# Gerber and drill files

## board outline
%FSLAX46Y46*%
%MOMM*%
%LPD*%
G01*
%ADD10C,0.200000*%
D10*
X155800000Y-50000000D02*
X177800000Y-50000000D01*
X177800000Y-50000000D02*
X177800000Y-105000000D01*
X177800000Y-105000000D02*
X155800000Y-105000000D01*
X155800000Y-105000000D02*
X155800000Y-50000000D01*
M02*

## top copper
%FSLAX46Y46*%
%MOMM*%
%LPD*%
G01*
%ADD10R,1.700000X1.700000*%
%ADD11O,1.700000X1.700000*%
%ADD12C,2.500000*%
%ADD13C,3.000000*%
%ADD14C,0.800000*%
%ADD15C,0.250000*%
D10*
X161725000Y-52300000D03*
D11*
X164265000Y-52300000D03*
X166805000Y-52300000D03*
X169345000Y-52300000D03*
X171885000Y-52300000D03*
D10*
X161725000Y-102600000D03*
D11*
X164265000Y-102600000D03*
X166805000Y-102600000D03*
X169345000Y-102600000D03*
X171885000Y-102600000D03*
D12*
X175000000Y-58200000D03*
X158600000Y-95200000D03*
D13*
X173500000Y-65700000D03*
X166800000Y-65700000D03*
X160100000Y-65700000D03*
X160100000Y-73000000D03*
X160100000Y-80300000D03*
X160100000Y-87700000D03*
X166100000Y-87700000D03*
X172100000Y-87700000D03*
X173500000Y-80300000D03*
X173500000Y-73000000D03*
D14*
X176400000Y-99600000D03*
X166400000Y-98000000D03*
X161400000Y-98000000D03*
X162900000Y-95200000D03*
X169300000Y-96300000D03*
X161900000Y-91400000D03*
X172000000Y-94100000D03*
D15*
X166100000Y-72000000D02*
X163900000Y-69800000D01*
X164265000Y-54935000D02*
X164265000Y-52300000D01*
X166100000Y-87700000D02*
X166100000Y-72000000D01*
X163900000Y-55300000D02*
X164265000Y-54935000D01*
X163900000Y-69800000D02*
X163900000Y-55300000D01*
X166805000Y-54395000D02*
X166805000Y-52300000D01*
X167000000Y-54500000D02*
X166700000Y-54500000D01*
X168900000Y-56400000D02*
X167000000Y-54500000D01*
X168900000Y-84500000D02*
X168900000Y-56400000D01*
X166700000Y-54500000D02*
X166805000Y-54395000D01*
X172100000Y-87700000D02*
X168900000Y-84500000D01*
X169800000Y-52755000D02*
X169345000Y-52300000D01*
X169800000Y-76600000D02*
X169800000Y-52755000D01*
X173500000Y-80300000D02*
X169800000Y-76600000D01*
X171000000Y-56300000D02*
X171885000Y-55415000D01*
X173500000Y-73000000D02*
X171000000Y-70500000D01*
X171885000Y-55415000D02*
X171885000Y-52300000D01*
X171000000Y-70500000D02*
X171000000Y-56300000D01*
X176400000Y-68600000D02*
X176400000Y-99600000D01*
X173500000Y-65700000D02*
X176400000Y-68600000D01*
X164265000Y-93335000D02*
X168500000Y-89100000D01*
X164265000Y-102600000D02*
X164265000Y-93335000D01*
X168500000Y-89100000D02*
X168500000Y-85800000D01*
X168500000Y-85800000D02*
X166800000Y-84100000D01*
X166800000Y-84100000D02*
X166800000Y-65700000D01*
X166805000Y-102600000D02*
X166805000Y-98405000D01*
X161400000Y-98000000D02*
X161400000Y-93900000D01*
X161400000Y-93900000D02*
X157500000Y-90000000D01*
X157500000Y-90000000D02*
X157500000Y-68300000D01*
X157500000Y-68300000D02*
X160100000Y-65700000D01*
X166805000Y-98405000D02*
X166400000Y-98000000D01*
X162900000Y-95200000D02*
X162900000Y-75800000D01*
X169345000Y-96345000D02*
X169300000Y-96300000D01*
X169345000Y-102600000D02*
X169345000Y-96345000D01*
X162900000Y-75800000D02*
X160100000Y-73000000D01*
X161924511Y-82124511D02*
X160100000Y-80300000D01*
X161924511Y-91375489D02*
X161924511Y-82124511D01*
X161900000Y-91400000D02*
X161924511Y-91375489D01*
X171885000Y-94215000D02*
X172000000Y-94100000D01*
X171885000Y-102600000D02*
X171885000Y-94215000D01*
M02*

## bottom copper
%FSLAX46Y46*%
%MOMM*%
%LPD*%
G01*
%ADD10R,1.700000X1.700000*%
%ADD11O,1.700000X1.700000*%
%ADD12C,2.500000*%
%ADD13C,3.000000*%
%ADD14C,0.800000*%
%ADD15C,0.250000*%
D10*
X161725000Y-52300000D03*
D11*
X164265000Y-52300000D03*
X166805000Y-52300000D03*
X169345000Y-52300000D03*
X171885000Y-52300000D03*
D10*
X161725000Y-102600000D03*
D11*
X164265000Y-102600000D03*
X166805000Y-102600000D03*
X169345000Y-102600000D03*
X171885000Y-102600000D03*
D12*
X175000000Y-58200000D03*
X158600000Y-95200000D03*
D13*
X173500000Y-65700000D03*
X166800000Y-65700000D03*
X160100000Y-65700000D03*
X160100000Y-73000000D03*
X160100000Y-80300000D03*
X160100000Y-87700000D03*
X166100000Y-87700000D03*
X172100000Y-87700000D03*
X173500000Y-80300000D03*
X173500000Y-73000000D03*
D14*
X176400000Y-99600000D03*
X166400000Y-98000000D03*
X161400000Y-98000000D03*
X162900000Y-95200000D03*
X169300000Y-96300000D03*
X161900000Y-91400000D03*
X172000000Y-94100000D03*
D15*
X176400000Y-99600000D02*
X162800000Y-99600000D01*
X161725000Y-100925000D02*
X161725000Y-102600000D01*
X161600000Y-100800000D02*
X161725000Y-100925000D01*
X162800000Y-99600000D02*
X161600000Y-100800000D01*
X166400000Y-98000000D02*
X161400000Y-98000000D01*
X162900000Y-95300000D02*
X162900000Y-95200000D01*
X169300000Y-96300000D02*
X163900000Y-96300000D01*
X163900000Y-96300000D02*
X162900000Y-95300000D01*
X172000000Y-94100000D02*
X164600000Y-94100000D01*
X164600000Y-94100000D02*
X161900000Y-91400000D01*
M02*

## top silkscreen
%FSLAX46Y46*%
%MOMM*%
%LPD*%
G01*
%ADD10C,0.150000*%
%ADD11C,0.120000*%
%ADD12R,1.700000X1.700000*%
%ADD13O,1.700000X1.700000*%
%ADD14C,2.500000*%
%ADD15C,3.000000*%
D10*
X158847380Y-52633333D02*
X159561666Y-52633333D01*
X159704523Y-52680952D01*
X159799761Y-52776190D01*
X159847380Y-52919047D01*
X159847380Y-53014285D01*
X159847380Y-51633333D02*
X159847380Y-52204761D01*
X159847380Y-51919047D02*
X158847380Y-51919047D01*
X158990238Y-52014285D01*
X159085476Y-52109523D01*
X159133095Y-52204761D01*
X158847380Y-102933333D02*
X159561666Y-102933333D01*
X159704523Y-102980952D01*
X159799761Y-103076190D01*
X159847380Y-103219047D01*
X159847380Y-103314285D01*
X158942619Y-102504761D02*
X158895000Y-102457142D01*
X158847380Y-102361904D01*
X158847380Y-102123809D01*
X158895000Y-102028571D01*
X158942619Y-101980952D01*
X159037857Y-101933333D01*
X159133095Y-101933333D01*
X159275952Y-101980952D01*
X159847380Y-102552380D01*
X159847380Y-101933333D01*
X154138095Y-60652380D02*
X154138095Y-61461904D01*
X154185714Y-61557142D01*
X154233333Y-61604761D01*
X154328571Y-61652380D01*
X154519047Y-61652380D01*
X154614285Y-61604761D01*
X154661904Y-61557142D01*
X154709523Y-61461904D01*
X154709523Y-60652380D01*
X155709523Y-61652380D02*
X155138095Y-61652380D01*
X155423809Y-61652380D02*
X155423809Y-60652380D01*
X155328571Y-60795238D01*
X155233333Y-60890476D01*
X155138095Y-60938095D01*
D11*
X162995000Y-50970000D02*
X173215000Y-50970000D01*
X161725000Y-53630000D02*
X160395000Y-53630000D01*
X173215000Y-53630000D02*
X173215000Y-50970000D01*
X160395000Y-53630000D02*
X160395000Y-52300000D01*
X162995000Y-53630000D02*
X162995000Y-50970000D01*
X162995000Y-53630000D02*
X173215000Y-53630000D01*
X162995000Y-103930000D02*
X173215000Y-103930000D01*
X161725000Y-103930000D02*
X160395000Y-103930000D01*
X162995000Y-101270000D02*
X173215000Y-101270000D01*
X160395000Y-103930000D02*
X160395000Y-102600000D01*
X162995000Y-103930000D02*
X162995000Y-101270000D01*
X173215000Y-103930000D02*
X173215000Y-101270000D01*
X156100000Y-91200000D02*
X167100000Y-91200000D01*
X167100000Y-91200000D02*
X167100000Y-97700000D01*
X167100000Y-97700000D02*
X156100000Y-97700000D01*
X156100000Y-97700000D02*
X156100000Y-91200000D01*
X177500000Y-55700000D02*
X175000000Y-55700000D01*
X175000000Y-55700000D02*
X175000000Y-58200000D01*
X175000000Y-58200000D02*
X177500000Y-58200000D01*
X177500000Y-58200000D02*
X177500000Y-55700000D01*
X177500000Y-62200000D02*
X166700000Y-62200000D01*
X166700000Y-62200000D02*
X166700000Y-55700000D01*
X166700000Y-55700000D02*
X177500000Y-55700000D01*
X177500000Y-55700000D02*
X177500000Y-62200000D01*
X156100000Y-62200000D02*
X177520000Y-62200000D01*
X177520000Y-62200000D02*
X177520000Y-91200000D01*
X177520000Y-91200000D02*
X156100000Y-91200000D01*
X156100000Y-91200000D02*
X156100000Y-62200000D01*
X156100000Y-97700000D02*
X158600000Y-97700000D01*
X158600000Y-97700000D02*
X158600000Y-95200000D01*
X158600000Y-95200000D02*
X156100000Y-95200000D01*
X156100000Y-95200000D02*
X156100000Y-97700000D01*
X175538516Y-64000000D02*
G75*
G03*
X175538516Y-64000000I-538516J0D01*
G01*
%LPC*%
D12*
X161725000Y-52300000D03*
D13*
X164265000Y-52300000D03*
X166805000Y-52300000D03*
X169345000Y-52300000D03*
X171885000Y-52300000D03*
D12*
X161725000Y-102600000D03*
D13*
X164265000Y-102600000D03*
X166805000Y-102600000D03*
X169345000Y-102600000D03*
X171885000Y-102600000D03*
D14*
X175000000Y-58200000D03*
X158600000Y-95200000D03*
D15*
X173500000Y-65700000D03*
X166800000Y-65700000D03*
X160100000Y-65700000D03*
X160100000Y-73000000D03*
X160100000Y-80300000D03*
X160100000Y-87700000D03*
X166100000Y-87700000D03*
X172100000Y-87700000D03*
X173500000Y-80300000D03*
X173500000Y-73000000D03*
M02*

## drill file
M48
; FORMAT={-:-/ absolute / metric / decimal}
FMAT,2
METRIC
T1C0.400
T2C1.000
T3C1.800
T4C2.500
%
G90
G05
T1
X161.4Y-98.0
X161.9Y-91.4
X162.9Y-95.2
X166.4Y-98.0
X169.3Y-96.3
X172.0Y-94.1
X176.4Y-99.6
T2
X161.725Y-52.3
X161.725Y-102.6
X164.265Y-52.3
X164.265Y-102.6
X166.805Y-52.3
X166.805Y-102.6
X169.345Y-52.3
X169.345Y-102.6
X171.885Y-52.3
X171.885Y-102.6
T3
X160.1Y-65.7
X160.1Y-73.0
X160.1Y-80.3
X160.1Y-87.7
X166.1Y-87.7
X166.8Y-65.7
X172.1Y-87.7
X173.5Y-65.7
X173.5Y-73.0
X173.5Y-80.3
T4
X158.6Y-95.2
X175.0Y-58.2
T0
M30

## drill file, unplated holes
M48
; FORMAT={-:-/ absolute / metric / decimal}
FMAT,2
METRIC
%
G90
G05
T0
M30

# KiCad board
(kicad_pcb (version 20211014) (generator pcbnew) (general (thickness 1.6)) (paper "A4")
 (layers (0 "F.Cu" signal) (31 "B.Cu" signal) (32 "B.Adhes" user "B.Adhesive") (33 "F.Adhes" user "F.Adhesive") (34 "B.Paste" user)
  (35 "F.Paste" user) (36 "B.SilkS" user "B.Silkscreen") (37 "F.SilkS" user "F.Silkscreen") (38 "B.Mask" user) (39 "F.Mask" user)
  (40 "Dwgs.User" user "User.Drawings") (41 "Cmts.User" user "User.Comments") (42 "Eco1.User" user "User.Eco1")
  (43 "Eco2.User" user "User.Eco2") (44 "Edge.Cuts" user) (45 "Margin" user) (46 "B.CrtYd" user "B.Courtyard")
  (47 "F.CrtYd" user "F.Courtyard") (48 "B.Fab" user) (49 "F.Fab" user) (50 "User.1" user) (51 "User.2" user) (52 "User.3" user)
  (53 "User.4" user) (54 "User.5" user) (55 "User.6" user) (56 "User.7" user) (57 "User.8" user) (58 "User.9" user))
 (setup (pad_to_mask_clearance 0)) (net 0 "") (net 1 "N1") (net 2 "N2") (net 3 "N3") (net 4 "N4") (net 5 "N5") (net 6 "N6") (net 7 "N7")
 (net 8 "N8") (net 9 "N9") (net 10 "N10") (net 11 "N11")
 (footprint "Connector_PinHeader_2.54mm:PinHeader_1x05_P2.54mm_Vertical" (layer "F.Cu") (at 161.725 52.3 90)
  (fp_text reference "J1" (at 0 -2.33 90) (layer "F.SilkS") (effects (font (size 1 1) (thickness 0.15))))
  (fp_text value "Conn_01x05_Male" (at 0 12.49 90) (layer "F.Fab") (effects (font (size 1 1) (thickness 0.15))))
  (fp_line (start 1.33 1.27) (end 1.33 11.49) (layer "F.SilkS") (width 0.12))
  (fp_line (start -1.33 0) (end -1.33 -1.33) (layer "F.SilkS") (width 0.12))
  (fp_line (start -1.33 11.49) (end 1.33 11.49) (layer "F.SilkS") (width 0.12))
  (fp_line (start -1.33 -1.33) (end 0 -1.33) (layer "F.SilkS") (width 0.12))
  (fp_line (start -1.33 1.27) (end 1.33 1.27) (layer "F.SilkS") (width 0.12))
  (fp_line (start -1.33 1.27) (end -1.33 11.49) (layer "F.SilkS") (width 0.12))
  (pad "1" thru_hole rect (at 0 0 90) (size 1.7 1.7) (drill 1) (layers *.Cu *.Mask) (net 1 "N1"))
  (pad "2" thru_hole oval (at 0 2.54 90) (size 1.7 1.7) (drill 1) (layers *.Cu *.Mask) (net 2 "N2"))
  (pad "3" thru_hole oval (at 0 5.08 90) (size 1.7 1.7) (drill 1) (layers *.Cu *.Mask) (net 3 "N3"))
  (pad "4" thru_hole oval (at 0 7.62 90) (size 1.7 1.7) (drill 1) (layers *.Cu *.Mask) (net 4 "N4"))
  (pad "5" thru_hole oval (at 0 10.16 90) (size 1.7 1.7) (drill 1) (layers *.Cu *.Mask) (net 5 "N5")))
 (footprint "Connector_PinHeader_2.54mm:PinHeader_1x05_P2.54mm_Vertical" (layer "F.Cu") (at 161.725 102.6 90)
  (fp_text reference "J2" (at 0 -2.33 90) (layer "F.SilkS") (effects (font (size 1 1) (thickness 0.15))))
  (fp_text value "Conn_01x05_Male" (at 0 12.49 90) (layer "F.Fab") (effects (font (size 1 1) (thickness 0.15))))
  (fp_line (start -1.33 1.27) (end -1.33 11.49) (layer "F.SilkS") (width 0.12))
  (fp_line (start -1.33 0) (end -1.33 -1.33) (layer "F.SilkS") (width 0.12))
  (fp_line (start 1.33 1.27) (end 1.33 11.49) (layer "F.SilkS") (width 0.12))
  (fp_line (start -1.33 -1.33) (end 0 -1.33) (layer "F.SilkS") (width 0.12))
  (fp_line (start -1.33 1.27) (end 1.33 1.27) (layer "F.SilkS") (width 0.12))
  (fp_line (start -1.33 11.49) (end 1.33 11.49) (layer "F.SilkS") (width 0.12))
  (pad "1" thru_hole rect (at 0 0 90) (size 1.7 1.7) (drill 1) (layers *.Cu *.Mask) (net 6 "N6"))
  (pad "2" thru_hole oval (at 0 2.54 90) (size 1.7 1.7) (drill 1) (layers *.Cu *.Mask) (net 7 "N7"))
  (pad "3" thru_hole oval (at 0 5.08 90) (size 1.7 1.7) (drill 1) (layers *.Cu *.Mask) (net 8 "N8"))
  (pad "4" thru_hole oval (at 0 7.62 90) (size 1.7 1.7) (drill 1) (layers *.Cu *.Mask) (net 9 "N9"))
  (pad "5" thru_hole oval (at 0 10.16 90) (size 1.7 1.7) (drill 1) (layers *.Cu *.Mask) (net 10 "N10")))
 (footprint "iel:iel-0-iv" (layer "F.Cu") (at 156.1 62.2)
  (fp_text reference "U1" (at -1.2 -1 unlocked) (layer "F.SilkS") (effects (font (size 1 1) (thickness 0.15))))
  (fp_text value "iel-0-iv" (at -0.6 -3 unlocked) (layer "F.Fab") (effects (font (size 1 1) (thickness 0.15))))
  (fp_rect (start 0 29) (end 11 35.5) (layer "F.SilkS") (width 0.12) (fill none))
  (fp_rect (start 21.4 -6.5) (end 18.9 -4) (layer "F.SilkS") (width 0.12) (fill none))
  (fp_rect (start 21.4 0) (end 10.6 -6.5) (layer "F.SilkS") (width 0.12) (fill none))
  (fp_rect (start 0 0) (end 21.42 29) (layer "F.SilkS") (width 0.12) (fill none))
  (fp_rect (start 0 35.5) (end 2.5 33) (layer "F.SilkS") (width 0.12) (fill none))
  (fp_circle (center 18.9 1.8) (end 19.4 2) (layer "F.SilkS") (width 0.12) (fill none))
  (pad "" thru_hole circle (at 18.9 -4) (size 2.5 2.5) (drill 2.5) (layers *.Cu *.Mask))
  (pad "" thru_hole circle (at 2.5 33) (size 2.5 2.5) (drill 2.5) (layers *.Cu *.Mask))
  (pad "0" thru_hole circle (at 17.4 3.5) (size 3 3) (drill 1.8) (layers *.Cu *.Mask) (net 6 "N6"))
  (pad "1" thru_hole circle (at 10.7 3.5) (size 3 3) (drill 1.8) (layers *.Cu *.Mask) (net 7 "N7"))
  (pad "2" thru_hole circle (at 4 3.5) (size 3 3) (drill 1.8) (layers *.Cu *.Mask) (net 8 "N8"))
  (pad "3" thru_hole circle (at 4 10.8) (size 3 3) (drill 1.8) (layers *.Cu *.Mask) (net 9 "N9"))
  (pad "4" thru_hole circle (at 4 18.1) (size 3 3) (drill 1.8) (layers *.Cu *.Mask) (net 10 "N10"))
  (pad "5" thru_hole circle (at 4 25.5) (size 3 3) (drill 1.8) (layers *.Cu *.Mask) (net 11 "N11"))
  (pad "6" thru_hole circle (at 10 25.5) (size 3 3) (drill 1.8) (layers *.Cu *.Mask) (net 2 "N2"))
  (pad "7" thru_hole circle (at 16 25.5) (size 3 3) (drill 1.8) (layers *.Cu *.Mask) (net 3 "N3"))
  (pad "8" thru_hole circle (at 17.4 18.1) (size 3 3) (drill 1.8) (layers *.Cu *.Mask) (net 4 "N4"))
  (pad "9" thru_hole circle (at 17.4 10.8) (size 3 3) (drill 1.8) (layers *.Cu *.Mask) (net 5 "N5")))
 (gr_rect (start 155.8 50) (end 177.8 105) (layer "Edge.Cuts") (width 0.2) (fill none))
 (segment (start 166.1 72) (end 163.9 69.8) (width 0.25) (layer "F.Cu") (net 2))
 (segment (start 164.265 54.935) (end 164.265 52.3) (width 0.25) (layer "F.Cu") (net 2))
 (segment (start 166.1 87.7) (end 166.1 72) (width 0.25) (layer "F.Cu") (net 2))
 (segment (start 163.9 55.3) (end 164.265 54.935) (width 0.25) (layer "F.Cu") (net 2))
 (segment (start 163.9 69.8) (end 163.9 55.3) (width 0.25) (layer "F.Cu") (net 2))
 (segment (start 166.805 54.395) (end 166.805 52.3) (width 0.25) (layer "F.Cu") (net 3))
 (segment (start 167 54.5) (end 166.7 54.5) (width 0.25) (layer "F.Cu") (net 3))
 (segment (start 168.9 56.4) (end 167 54.5) (width 0.25) (layer "F.Cu") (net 3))
 (segment (start 168.9 84.5) (end 168.9 56.4) (width 0.25) (layer "F.Cu") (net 3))
 (segment (start 166.7 54.5) (end 166.805 54.395) (width 0.25) (layer "F.Cu") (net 3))
 (segment (start 172.1 87.7) (end 168.9 84.5) (width 0.25) (layer "F.Cu") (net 3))
 (segment (start 169.8 52.755) (end 169.345 52.3) (width 0.25) (layer "F.Cu") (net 4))
 (segment (start 169.8 76.6) (end 169.8 52.755) (width 0.25) (layer "F.Cu") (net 4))
 (segment (start 173.5 80.3) (end 169.8 76.6) (width 0.25) (layer "F.Cu") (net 4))
 (segment (start 171 56.3) (end 171.885 55.415) (width 0.25) (layer "F.Cu") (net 5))
 (segment (start 173.5 73) (end 171 70.5) (width 0.25) (layer "F.Cu") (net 5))
 (segment (start 171.885 55.415) (end 171.885 52.3) (width 0.25) (layer "F.Cu") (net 5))
 (segment (start 171 70.5) (end 171 56.3) (width 0.25) (layer "F.Cu") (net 5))
 (segment (start 176.4 68.6) (end 176.4 99.6) (width 0.25) (layer "F.Cu") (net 6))
 (segment (start 173.5 65.7) (end 176.4 68.6) (width 0.25) (layer "F.Cu") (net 6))
 (via (at 176.4 99.6) (size 0.8) (drill 0.4) (layers "F.Cu" "B.Cu") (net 6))
 (segment (start 176.4 99.6) (end 162.8 99.6) (width 0.25) (layer "B.Cu") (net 6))
 (segment (start 161.725 100.925) (end 161.725 102.6) (width 0.25) (layer "B.Cu") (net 6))
 (segment (start 161.6 100.8) (end 161.725 100.925) (width 0.25) (layer "B.Cu") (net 6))
 (segment (start 162.8 99.6) (end 161.6 100.8) (width 0.25) (layer "B.Cu") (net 6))
 (segment (start 164.265 93.335) (end 168.5 89.1) (width 0.25) (layer "F.Cu") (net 7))
 (segment (start 164.265 102.6) (end 164.265 93.335) (width 0.25) (layer "F.Cu") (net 7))
 (segment (start 168.5 89.1) (end 168.5 85.8) (width 0.25) (layer "F.Cu") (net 7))
 (segment (start 168.5 85.8) (end 166.8 84.1) (width 0.25) (layer "F.Cu") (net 7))
 (segment (start 166.8 84.1) (end 166.8 65.7) (width 0.25) (layer "F.Cu") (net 7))
 (segment (start 166.805 102.6) (end 166.805 98.405) (width 0.25) (layer "F.Cu") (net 8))
 (segment (start 161.4 98) (end 161.4 93.9) (width 0.25) (layer "F.Cu") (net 8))
 (segment (start 161.4 93.9) (end 157.5 90) (width 0.25) (layer "F.Cu") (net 8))
 (segment (start 157.5 90) (end 157.5 68.3) (width 0.25) (layer "F.Cu") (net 8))
 (segment (start 157.5 68.3) (end 160.1 65.7) (width 0.25) (layer "F.Cu") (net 8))
 (segment (start 166.805 98.405) (end 166.4 98) (width 0.25) (layer "F.Cu") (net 8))
 (via (at 166.4 98) (size 0.8) (drill 0.4) (layers "F.Cu" "B.Cu") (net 8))
 (via (at 161.4 98) (size 0.8) (drill 0.4) (layers "F.Cu" "B.Cu") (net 8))
 (segment (start 166.4 98) (end 161.4 98) (width 0.25) (layer "B.Cu") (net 8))
 (segment (start 162.9 95.2) (end 162.9 75.8) (width 0.25) (layer "F.Cu") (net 9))
 (segment (start 169.345 96.345) (end 169.3 96.3) (width 0.25) (layer "F.Cu") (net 9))
 (segment (start 169.345 102.6) (end 169.345 96.345) (width 0.25) (layer "F.Cu") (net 9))
 (segment (start 162.9 75.8) (end 160.1 73) (width 0.25) (layer "F.Cu") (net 9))
 (via (at 162.9 95.2) (size 0.8) (drill 0.4) (layers "F.Cu" "B.Cu") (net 9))
 (via (at 169.3 96.3) (size 0.8) (drill 0.4) (layers "F.Cu" "B.Cu") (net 9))
 (segment (start 162.9 95.3) (end 162.9 95.2) (width 0.25) (layer "B.Cu") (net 9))
 (segment (start 169.3 96.3) (end 163.9 96.3) (width 0.25) (layer "B.Cu") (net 9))
 (segment (start 163.9 96.3) (end 162.9 95.3) (width 0.25) (layer "B.Cu") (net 9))
 (segment (start 161.924511 82.124511) (end 160.1 80.3) (width 0.25) (layer "F.Cu") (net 10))
 (segment (start 161.924511 91.375489) (end 161.924511 82.124511) (width 0.25) (layer "F.Cu") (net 10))
 (segment (start 161.9 91.4) (end 161.924511 91.375489) (width 0.25) (layer "F.Cu") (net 10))
 (segment (start 171.885 94.215) (end 172 94.1) (width 0.25) (layer "F.Cu") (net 10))
 (segment (start 171.885 102.6) (end 171.885 94.215) (width 0.25) (layer "F.Cu") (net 10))
 (via (at 161.9 91.4) (size 0.8) (drill 0.4) (layers "F.Cu" "B.Cu") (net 10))
 (via (at 172 94.1) (size 0.8) (drill 0.4) (layers "F.Cu" "B.Cu") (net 10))
 (segment (start 172 94.1) (end 164.6 94.1) (width 0.25) (layer "B.Cu") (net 10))
 (segment (start 164.6 94.1) (end 161.9 91.4) (width 0.25) (layer "B.Cu") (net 10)))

